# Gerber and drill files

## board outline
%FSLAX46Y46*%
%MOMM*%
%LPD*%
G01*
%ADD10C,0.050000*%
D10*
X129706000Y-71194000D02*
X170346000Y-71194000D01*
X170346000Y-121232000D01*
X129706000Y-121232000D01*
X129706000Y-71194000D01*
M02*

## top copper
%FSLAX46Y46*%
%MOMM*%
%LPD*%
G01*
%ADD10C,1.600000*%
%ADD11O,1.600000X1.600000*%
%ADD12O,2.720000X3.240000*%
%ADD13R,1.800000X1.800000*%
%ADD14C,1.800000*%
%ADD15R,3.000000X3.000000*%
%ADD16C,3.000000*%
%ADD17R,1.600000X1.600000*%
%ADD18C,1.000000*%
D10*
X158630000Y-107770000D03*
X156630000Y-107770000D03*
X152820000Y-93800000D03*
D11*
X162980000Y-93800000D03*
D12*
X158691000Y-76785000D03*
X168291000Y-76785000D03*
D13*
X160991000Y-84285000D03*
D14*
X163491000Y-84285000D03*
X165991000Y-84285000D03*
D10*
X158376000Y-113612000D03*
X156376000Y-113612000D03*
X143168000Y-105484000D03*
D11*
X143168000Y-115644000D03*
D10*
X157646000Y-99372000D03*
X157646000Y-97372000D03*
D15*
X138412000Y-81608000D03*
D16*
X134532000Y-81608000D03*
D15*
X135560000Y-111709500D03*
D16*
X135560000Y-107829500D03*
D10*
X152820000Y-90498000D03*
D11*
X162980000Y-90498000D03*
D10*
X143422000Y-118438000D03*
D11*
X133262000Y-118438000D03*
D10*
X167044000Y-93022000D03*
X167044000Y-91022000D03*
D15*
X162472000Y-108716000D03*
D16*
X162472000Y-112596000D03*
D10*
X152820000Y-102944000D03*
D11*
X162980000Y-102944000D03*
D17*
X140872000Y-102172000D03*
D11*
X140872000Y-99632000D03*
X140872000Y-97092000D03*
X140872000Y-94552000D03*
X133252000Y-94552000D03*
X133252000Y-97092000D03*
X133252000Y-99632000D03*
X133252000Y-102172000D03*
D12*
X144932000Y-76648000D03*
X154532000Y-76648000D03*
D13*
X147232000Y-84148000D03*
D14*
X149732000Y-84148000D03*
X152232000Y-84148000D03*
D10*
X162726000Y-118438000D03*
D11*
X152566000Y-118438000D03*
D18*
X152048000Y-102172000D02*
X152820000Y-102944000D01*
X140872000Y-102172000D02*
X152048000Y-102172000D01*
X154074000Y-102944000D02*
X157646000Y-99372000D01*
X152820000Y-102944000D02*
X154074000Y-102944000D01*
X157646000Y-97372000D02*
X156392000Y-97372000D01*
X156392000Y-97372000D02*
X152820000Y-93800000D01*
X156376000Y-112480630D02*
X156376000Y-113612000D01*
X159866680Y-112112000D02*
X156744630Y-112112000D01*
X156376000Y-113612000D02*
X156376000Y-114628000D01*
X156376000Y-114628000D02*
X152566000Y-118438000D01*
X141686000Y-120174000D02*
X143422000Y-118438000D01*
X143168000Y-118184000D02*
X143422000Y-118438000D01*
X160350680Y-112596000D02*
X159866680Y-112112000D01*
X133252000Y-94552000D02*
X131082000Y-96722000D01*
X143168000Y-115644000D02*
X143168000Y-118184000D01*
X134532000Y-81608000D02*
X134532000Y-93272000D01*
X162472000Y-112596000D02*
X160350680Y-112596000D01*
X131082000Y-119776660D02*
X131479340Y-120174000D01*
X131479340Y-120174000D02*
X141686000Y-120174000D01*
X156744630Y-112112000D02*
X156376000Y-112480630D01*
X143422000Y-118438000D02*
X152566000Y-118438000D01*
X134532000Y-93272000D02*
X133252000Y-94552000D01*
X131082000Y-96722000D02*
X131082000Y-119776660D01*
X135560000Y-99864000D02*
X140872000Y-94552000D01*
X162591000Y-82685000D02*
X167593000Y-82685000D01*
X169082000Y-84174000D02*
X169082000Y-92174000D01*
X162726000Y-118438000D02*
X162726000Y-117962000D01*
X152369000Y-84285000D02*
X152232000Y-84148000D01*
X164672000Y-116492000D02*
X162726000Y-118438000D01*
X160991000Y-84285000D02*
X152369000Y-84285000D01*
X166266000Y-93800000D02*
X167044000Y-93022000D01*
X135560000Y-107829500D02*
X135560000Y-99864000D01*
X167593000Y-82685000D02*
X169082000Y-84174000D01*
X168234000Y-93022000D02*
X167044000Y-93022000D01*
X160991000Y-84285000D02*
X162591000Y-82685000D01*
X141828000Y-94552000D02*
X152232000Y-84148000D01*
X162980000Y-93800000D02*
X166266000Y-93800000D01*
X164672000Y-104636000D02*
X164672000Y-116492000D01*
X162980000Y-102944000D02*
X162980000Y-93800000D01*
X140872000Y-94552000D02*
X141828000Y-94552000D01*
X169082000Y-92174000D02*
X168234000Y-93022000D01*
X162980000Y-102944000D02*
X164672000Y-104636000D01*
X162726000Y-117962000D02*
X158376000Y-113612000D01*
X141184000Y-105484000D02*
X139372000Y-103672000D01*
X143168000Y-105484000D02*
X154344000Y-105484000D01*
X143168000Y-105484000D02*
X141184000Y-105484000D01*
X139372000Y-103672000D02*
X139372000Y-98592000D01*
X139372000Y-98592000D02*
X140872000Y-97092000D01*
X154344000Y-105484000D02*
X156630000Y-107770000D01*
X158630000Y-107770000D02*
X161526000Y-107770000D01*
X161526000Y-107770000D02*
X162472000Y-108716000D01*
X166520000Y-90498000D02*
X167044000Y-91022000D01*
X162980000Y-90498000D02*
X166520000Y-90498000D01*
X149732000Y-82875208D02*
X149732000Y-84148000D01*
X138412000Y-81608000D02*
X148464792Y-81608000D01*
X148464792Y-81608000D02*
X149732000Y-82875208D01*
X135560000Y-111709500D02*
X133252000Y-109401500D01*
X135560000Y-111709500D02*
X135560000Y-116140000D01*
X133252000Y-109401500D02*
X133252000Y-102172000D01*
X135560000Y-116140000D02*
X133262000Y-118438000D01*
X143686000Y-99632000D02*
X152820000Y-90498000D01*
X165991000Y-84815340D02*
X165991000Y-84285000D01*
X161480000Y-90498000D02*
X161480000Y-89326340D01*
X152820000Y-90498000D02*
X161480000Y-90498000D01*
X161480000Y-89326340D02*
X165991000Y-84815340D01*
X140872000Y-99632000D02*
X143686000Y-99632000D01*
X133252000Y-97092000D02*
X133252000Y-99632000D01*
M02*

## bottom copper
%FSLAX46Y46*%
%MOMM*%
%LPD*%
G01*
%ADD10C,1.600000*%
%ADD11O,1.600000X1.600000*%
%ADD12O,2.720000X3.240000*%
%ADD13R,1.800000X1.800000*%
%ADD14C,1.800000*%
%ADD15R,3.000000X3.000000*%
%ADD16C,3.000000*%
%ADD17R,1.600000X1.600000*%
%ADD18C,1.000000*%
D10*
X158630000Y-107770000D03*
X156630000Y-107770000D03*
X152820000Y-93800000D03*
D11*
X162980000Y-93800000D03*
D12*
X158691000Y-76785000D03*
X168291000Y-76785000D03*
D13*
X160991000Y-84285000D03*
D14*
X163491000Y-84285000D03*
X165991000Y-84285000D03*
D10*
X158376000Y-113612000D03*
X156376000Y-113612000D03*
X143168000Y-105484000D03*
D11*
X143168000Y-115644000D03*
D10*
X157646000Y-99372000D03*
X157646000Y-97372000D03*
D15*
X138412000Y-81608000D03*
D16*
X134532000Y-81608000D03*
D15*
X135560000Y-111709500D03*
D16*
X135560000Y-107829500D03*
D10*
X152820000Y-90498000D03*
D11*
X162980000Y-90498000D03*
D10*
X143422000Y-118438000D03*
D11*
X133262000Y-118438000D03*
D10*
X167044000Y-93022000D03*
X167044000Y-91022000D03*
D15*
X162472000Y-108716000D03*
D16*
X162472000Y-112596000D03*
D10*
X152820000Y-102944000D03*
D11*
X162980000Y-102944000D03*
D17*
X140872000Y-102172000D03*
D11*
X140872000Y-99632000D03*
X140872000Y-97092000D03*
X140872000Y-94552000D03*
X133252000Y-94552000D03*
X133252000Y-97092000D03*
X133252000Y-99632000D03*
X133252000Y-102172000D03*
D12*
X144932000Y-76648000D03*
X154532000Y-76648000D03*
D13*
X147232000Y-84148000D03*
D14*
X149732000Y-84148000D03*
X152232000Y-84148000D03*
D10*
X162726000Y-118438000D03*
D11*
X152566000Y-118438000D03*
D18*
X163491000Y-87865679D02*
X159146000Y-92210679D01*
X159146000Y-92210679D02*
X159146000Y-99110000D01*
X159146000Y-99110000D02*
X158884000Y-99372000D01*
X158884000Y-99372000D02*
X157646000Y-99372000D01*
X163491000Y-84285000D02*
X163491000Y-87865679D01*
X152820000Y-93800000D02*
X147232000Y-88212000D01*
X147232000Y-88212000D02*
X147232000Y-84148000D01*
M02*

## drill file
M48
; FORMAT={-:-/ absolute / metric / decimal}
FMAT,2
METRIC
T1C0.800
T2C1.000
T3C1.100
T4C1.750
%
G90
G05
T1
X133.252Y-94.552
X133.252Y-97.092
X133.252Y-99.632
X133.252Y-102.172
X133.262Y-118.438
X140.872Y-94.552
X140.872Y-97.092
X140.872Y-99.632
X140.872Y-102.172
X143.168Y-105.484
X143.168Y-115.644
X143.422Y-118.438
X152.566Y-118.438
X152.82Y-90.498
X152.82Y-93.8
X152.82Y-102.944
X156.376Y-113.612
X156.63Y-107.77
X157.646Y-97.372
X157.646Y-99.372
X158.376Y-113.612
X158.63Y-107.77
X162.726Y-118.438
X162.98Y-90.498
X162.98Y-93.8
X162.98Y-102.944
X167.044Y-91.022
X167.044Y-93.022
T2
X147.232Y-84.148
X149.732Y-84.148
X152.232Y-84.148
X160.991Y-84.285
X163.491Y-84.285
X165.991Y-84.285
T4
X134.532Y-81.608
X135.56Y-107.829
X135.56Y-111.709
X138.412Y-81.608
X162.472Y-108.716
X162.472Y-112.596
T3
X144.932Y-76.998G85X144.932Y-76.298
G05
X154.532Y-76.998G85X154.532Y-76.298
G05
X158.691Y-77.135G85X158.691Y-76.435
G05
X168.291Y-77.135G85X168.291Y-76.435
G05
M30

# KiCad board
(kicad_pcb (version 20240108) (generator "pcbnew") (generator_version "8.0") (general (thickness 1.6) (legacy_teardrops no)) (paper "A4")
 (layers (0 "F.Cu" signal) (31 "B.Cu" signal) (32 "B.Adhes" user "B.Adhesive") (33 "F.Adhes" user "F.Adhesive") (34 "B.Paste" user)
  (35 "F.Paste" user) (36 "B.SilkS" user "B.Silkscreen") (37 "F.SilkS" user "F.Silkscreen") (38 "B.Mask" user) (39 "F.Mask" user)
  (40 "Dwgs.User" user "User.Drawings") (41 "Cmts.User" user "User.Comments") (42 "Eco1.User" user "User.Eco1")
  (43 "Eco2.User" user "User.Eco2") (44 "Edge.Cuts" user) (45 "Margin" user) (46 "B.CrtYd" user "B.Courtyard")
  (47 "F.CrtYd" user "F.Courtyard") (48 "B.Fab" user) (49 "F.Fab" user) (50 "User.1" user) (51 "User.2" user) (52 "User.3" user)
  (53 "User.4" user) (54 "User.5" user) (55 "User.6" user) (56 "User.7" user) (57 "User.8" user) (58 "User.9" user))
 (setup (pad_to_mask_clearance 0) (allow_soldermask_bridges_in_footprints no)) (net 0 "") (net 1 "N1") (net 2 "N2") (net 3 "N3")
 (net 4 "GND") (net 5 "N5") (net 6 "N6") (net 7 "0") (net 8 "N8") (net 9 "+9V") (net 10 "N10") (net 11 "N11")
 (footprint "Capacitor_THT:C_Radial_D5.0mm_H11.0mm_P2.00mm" (layer "F.Cu") (at 158.63 107.77 180)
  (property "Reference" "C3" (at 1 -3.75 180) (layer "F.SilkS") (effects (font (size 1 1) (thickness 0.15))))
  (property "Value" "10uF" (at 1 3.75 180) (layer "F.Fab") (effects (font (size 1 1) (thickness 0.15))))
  (pad "1" thru_hole circle (at 0 0 180) (size 1.6 1.6) (drill 0.8) (layers "*.Cu" "*.Mask") (remove_unused_layers no) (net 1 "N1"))
  (pad "2" thru_hole circle (at 2 0 180) (size 1.6 1.6) (drill 0.8) (layers "*.Cu" "*.Mask") (remove_unused_layers no) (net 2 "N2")))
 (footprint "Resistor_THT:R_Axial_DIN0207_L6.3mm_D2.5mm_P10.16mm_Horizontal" (layer "F.Cu") (at 152.82 93.8)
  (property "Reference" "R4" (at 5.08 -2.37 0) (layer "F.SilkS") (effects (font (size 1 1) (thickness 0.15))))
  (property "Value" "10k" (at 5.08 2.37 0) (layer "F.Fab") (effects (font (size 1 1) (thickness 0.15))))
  (pad "1" thru_hole circle (at 0 0) (size 1.6 1.6) (drill 0.8) (layers "*.Cu" "*.Mask") (remove_unused_layers no) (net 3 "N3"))
  (pad "2" thru_hole oval (at 10.16 0) (size 1.6 1.6) (drill 0.8) (layers "*.Cu" "*.Mask") (remove_unused_layers no) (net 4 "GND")))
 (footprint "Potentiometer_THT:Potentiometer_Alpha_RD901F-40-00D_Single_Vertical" (layer "F.Cu") (at 160.991 84.285 90)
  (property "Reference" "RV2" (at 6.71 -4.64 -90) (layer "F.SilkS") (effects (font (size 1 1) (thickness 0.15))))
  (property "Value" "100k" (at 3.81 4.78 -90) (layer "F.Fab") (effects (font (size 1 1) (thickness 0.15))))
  (pad "" thru_hole oval (at 7.5 -2.3 180) (size 2.72 3.24) (drill oval 1.1 1.8) (layers "*.Cu" "*.Mask") (remove_unused_layers no))
  (pad "" thru_hole oval (at 7.5 7.3 180) (size 2.72 3.24) (drill oval 1.1 1.8) (layers "*.Cu" "*.Mask") (remove_unused_layers no))
  (pad "1" thru_hole rect (at 0 0 180) (size 1.8 1.8) (drill 1) (layers "*.Cu" "*.Mask") (remove_unused_layers no) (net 4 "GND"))
  (pad "2" thru_hole circle (at 0 2.5 180) (size 1.8 1.8) (drill 1) (layers "*.Cu" "*.Mask") (remove_unused_layers no) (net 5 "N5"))
  (pad "3" thru_hole circle (at 0 5 180) (size 1.8 1.8) (drill 1) (layers "*.Cu" "*.Mask") (remove_unused_layers no) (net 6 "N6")))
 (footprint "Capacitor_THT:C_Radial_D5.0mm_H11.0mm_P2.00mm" (layer "F.Cu") (at 158.376 113.612 180)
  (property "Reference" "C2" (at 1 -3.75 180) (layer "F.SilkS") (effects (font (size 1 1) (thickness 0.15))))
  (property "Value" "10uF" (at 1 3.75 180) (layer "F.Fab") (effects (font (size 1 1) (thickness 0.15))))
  (pad "1" thru_hole circle (at 0 0 180) (size 1.6 1.6) (drill 0.8) (layers "*.Cu" "*.Mask") (remove_unused_layers no) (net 4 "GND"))
  (pad "2" thru_hole circle (at 2 0 180) (size 1.6 1.6) (drill 0.8) (layers "*.Cu" "*.Mask") (remove_unused_layers no) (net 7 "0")))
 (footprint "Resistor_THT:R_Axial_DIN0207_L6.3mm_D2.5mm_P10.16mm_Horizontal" (layer "F.Cu") (at 143.168 105.484 -90)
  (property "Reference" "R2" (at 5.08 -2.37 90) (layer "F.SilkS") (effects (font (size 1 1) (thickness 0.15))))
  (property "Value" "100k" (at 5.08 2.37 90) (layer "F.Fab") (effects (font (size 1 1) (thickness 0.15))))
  (pad "1" thru_hole circle (at 0 0 270) (size 1.6 1.6) (drill 0.8) (layers "*.Cu" "*.Mask") (remove_unused_layers no) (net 2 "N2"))
  (pad "2" thru_hole oval (at 10.16 0 270) (size 1.6 1.6) (drill 0.8) (layers "*.Cu" "*.Mask") (remove_unused_layers no) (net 7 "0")))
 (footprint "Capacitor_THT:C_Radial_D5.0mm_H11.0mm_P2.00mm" (layer "F.Cu") (at 157.646 99.372 90)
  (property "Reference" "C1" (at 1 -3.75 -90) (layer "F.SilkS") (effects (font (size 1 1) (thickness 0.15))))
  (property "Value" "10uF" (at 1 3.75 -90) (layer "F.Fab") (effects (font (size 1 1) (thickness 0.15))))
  (pad "1" thru_hole circle (at 0 0 90) (size 1.6 1.6) (drill 0.8) (layers "*.Cu" "*.Mask") (remove_unused_layers no) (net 5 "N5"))
  (pad "2" thru_hole circle (at 2 0 90) (size 1.6 1.6) (drill 0.8) (layers "*.Cu" "*.Mask") (remove_unused_layers no) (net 3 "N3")))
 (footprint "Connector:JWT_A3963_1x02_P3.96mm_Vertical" (layer "F.Cu") (at 138.412 81.608 180)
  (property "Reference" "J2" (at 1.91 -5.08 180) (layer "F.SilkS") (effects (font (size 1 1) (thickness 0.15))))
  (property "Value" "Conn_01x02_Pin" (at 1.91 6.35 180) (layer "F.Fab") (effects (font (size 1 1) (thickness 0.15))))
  (pad "1" thru_hole rect (at 0 0 180) (size 3 3) (drill 1.75) (layers "*.Cu" "*.Mask") (remove_unused_layers no) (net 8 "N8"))
  (pad "2" thru_hole circle (at 3.88 0 180) (size 3 3) (drill 1.75) (layers "*.Cu" "*.Mask") (remove_unused_layers no) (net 7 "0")))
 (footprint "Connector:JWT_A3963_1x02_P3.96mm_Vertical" (layer "F.Cu") (at 135.56 111.7095 90)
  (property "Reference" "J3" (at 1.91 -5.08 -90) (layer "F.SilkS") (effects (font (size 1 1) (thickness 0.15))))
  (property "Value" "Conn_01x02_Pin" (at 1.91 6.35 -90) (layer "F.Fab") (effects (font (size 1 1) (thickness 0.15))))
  (pad "1" thru_hole rect (at 0 0 90) (size 3 3) (drill 1.75) (layers "*.Cu" "*.Mask") (remove_unused_layers no) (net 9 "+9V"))
  (pad "2" thru_hole circle (at 3.88 0 90) (size 3 3) (drill 1.75) (layers "*.Cu" "*.Mask") (remove_unused_layers no) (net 4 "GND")))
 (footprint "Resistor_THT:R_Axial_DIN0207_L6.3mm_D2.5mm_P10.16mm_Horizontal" (layer "F.Cu") (at 152.82 90.498)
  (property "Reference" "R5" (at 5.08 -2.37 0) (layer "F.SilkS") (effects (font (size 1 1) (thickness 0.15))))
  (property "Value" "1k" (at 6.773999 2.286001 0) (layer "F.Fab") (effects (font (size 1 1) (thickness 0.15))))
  (pad "1" thru_hole circle (at 0 0) (size 1.6 1.6) (drill 0.8) (layers "*.Cu" "*.Mask") (remove_unused_layers no) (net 6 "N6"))
  (pad "2" thru_hole oval (at 10.16 0) (size 1.6 1.6) (drill 0.8) (layers "*.Cu" "*.Mask") (remove_unused_layers no) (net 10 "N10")))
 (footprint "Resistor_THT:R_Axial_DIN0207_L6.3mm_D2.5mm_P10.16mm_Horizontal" (layer "F.Cu") (at 143.422 118.438 180)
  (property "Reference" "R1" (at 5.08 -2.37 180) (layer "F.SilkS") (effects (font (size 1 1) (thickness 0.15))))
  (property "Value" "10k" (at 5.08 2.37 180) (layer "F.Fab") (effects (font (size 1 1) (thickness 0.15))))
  (pad "1" thru_hole circle (at 0 0 180) (size 1.6 1.6) (drill 0.8) (layers "*.Cu" "*.Mask") (remove_unused_layers no) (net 7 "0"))
  (pad "2" thru_hole oval (at 10.16 0 180) (size 1.6 1.6) (drill 0.8) (layers "*.Cu" "*.Mask") (remove_unused_layers no) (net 9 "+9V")))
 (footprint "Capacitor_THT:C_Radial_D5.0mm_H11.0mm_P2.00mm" (layer "F.Cu") (at 167.044 93.022 90)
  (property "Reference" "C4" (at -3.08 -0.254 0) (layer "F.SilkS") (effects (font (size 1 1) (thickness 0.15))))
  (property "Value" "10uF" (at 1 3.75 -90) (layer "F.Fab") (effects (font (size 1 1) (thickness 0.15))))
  (pad "1" thru_hole circle (at 0 0 90) (size 1.6 1.6) (drill 0.8) (layers "*.Cu" "*.Mask") (remove_unused_layers no) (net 4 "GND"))
  (pad "2" thru_hole circle (at 2 0 90) (size 1.6 1.6) (drill 0.8) (layers "*.Cu" "*.Mask") (remove_unused_layers no) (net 10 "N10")))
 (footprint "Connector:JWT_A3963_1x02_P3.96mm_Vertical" (layer "F.Cu") (at 162.472 108.716 -90)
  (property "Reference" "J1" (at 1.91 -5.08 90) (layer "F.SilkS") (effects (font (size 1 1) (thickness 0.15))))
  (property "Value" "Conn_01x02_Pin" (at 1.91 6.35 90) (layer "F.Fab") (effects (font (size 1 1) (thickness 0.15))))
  (pad "1" thru_hole rect (at 0 0 270) (size 3 3) (drill 1.75) (layers "*.Cu" "*.Mask") (remove_unused_layers no) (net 1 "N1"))
  (pad "2" thru_hole circle (at 3.88 0 270) (size 3 3) (drill 1.75) (layers "*.Cu" "*.Mask") (remove_unused_layers no) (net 7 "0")))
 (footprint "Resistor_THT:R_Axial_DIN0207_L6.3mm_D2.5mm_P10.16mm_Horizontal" (layer "F.Cu") (at 152.82 102.944)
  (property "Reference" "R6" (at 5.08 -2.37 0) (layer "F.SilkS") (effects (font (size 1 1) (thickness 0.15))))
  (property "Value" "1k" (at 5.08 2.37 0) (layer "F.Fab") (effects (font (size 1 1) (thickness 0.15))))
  (pad "1" thru_hole circle (at 0 0) (size 1.6 1.6) (drill 0.8) (layers "*.Cu" "*.Mask") (remove_unused_layers no) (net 5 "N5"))
  (pad "2" thru_hole oval (at 10.16 0) (size 1.6 1.6) (drill 0.8) (layers "*.Cu" "*.Mask") (remove_unused_layers no) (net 4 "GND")))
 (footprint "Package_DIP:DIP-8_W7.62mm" (layer "F.Cu") (at 140.872 102.172 180)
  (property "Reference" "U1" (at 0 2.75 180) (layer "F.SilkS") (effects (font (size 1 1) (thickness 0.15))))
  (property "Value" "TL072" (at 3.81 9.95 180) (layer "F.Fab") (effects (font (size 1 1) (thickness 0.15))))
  (pad "1" thru_hole rect (at 0 0 180) (size 1.6 1.6) (drill 0.8) (layers "*.Cu" "*.Mask") (remove_unused_layers no) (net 5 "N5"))
  (pad "2" thru_hole oval (at 0 2.54 180) (size 1.6 1.6) (drill 0.8) (layers "*.Cu" "*.Mask") (remove_unused_layers no) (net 6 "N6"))
  (pad "3" thru_hole oval (at 0 5.08 180) (size 1.6 1.6) (drill 0.8) (layers "*.Cu" "*.Mask") (remove_unused_layers no) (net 2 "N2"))
  (pad "4" thru_hole oval (at 0 7.62 180) (size 1.6 1.6) (drill 0.8) (layers "*.Cu" "*.Mask") (remove_unused_layers no) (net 4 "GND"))
  (pad "5" thru_hole oval (at 7.62 7.62 180) (size 1.6 1.6) (drill 0.8) (layers "*.Cu" "*.Mask") (remove_unused_layers no) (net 7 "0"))
  (pad "6" thru_hole oval (at 7.62 5.08 180) (size 1.6 1.6) (drill 0.8) (layers "*.Cu" "*.Mask") (remove_unused_layers no) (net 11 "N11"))
  (pad "7" thru_hole oval (at 7.62 2.54 180) (size 1.6 1.6) (drill 0.8) (layers "*.Cu" "*.Mask") (remove_unused_layers no) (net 11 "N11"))
  (pad "8" thru_hole oval (at 7.62 0 180) (size 1.6 1.6) (drill 0.8) (layers "*.Cu" "*.Mask") (remove_unused_layers no) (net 9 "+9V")))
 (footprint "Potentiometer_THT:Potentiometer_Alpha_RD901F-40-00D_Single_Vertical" (layer "F.Cu") (at 147.232 84.148 90)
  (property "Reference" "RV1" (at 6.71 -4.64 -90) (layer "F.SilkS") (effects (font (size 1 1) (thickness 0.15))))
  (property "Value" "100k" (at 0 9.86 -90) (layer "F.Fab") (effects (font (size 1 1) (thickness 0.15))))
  (pad "" thru_hole oval (at 7.5 -2.3 180) (size 2.72 3.24) (drill oval 1.1 1.8) (layers "*.Cu" "*.Mask") (remove_unused_layers no))
  (pad "" thru_hole oval (at 7.5 7.3 180) (size 2.72 3.24) (drill oval 1.1 1.8) (layers "*.Cu" "*.Mask") (remove_unused_layers no))
  (pad "1" thru_hole rect (at 0 0 180) (size 1.8 1.8) (drill 1) (layers "*.Cu" "*.Mask") (remove_unused_layers no) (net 3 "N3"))
  (pad "2" thru_hole circle (at 0 2.5 180) (size 1.8 1.8) (drill 1) (layers "*.Cu" "*.Mask") (remove_unused_layers no) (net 8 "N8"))
  (pad "3" thru_hole circle (at 0 5 180) (size 1.8 1.8) (drill 1) (layers "*.Cu" "*.Mask") (remove_unused_layers no) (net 4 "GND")))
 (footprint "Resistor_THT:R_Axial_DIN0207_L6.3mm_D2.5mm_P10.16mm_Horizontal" (layer "F.Cu") (at 162.726 118.438 180)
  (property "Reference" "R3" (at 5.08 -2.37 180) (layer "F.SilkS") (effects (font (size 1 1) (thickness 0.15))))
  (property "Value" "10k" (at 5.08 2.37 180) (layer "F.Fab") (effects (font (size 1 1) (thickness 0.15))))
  (pad "1" thru_hole circle (at 0 0 180) (size 1.6 1.6) (drill 0.8) (layers "*.Cu" "*.Mask") (remove_unused_layers no) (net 4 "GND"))
  (pad "2" thru_hole oval (at 10.16 0 180) (size 1.6 1.6) (drill 0.8) (layers "*.Cu" "*.Mask") (remove_unused_layers no) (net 7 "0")))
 (gr_rect (start 129.706 71.194) (end 170.346 121.232) (stroke (width 0.05) (type default)) (fill none) (layer "Edge.Cuts"))
 (segment (start 152.048 102.172) (end 152.82 102.944) (width 1) (layer "F.Cu") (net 5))
 (segment (start 140.872 102.172) (end 152.048 102.172) (width 1) (layer "F.Cu") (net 5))
 (segment (start 154.074 102.944) (end 157.646 99.372) (width 1) (layer "F.Cu") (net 5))
 (segment (start 152.82 102.944) (end 154.074 102.944) (width 1) (layer "F.Cu") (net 5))
 (segment (start 163.491 87.865679) (end 159.146 92.210679) (width 1) (layer "B.Cu") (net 5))
 (segment (start 159.146 92.210679) (end 159.146 99.11) (width 1) (layer "B.Cu") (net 5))
 (segment (start 159.146 99.11) (end 158.884 99.372) (width 1) (layer "B.Cu") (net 5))
 (segment (start 158.884 99.372) (end 157.646 99.372) (width 1) (layer "B.Cu") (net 5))
 (segment (start 163.491 84.285) (end 163.491 87.865679) (width 1) (layer "B.Cu") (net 5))
 (segment (start 157.646 97.372) (end 156.392 97.372) (width 1) (layer "F.Cu") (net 3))
 (segment (start 156.392 97.372) (end 152.82 93.8) (width 1) (layer "F.Cu") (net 3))
 (segment (start 152.82 93.8) (end 147.232 88.212) (width 1) (layer "B.Cu") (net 3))
 (segment (start 147.232 88.212) (end 147.232 84.148) (width 1) (layer "B.Cu") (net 3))
 (segment (start 156.376 112.48063) (end 156.376 113.612) (width 1) (layer "F.Cu") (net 7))
 (segment (start 159.86668 112.112) (end 156.74463 112.112) (width 1) (layer "F.Cu") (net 7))
 (segment (start 156.376 113.612) (end 156.376 114.628) (width 1) (layer "F.Cu") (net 7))
 (segment (start 156.376 114.628) (end 152.566 118.438) (width 1) (layer "F.Cu") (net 7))
 (segment (start 141.686 120.174) (end 143.422 118.438) (width 1) (layer "F.Cu") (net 7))
 (segment (start 143.168 118.184) (end 143.422 118.438) (width 1) (layer "F.Cu") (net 7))
 (segment (start 160.35068 112.596) (end 159.86668 112.112) (width 1) (layer "F.Cu") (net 7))
 (segment (start 133.252 94.552) (end 131.082 96.722) (width 1) (layer "F.Cu") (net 7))
 (segment (start 143.168 115.644) (end 143.168 118.184) (width 1) (layer "F.Cu") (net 7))
 (segment (start 134.532 81.608) (end 134.532 93.272) (width 1) (layer "F.Cu") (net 7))
 (segment (start 162.472 112.596) (end 160.35068 112.596) (width 1) (layer "F.Cu") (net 7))
 (segment (start 131.082 119.77666) (end 131.47934 120.174) (width 1) (layer "F.Cu") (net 7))
 (segment (start 131.47934 120.174) (end 141.686 120.174) (width 1) (layer "F.Cu") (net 7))
 (segment (start 156.74463 112.112) (end 156.376 112.48063) (width 1) (layer "F.Cu") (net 7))
 (segment (start 143.422 118.438) (end 152.566 118.438) (width 1) (layer "F.Cu") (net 7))
 (segment (start 134.532 93.272) (end 133.252 94.552) (width 1) (layer "F.Cu") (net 7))
 (segment (start 131.082 96.722) (end 131.082 119.77666) (width 1) (layer "F.Cu") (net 7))
 (segment (start 135.56 99.864) (end 140.872 94.552) (width 1) (layer "F.Cu") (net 4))
 (segment (start 162.591 82.685) (end 167.593 82.685) (width 1) (layer "F.Cu") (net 4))
 (segment (start 169.082 84.174) (end 169.082 92.174) (width 1) (layer "F.Cu") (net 4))
 (segment (start 162.726 118.438) (end 162.726 117.962) (width 1) (layer "F.Cu") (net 4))
 (segment (start 152.369 84.285) (end 152.232 84.148) (width 1) (layer "F.Cu") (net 4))
 (segment (start 164.672 116.492) (end 162.726 118.438) (width 1) (layer "F.Cu") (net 4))
 (segment (start 160.991 84.285) (end 152.369 84.285) (width 1) (layer "F.Cu") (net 4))
 (segment (start 166.266 93.8) (end 167.044 93.022) (width 1) (layer "F.Cu") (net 4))
 (segment (start 135.56 107.8295) (end 135.56 99.864) (width 1) (layer "F.Cu") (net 4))
 (segment (start 167.593 82.685) (end 169.082 84.174) (width 1) (layer "F.Cu") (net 4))
 (segment (start 168.234 93.022) (end 167.044 93.022) (width 1) (layer "F.Cu") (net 4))
 (segment (start 160.991 84.285) (end 162.591 82.685) (width 1) (layer "F.Cu") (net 4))
 (segment (start 141.828 94.552) (end 152.232 84.148) (width 1) (layer "F.Cu") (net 4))
 (segment (start 162.98 93.8) (end 166.266 93.8) (width 1) (layer "F.Cu") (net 4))
 (segment (start 164.672 104.636) (end 164.672 116.492) (width 1) (layer "F.Cu") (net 4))
 (segment (start 162.98 102.944) (end 162.98 93.8) (width 1) (layer "F.Cu") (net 4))
 (segment (start 140.872 94.552) (end 141.828 94.552) (width 1) (layer "F.Cu") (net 4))
 (segment (start 169.082 92.174) (end 168.234 93.022) (width 1) (layer "F.Cu") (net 4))
 (segment (start 162.98 102.944) (end 164.672 104.636) (width 1) (layer "F.Cu") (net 4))
 (segment (start 162.726 117.962) (end 158.376 113.612) (width 1) (layer "F.Cu") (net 4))
 (segment (start 141.184 105.484) (end 139.372 103.672) (width 1) (layer "F.Cu") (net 2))
 (segment (start 143.168 105.484) (end 154.344 105.484) (width 1) (layer "F.Cu") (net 2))
 (segment (start 143.168 105.484) (end 141.184 105.484) (width 1) (layer "F.Cu") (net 2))
 (segment (start 139.372 103.672) (end 139.372 98.592) (width 1) (layer "F.Cu") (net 2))
 (segment (start 139.372 98.592) (end 140.872 97.092) (width 1) (layer "F.Cu") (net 2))
 (segment (start 154.344 105.484) (end 156.63 107.77) (width 1) (layer "F.Cu") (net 2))
 (segment (start 158.63 107.77) (end 161.526 107.77) (width 1) (layer "F.Cu") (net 1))
 (segment (start 161.526 107.77) (end 162.472 108.716) (width 1) (layer "F.Cu") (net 1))
 (segment (start 166.52 90.498) (end 167.044 91.022) (width 1) (layer "F.Cu") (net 10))
 (segment (start 162.98 90.498) (end 166.52 90.498) (width 1) (layer "F.Cu") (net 10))
 (segment (start 149.732 82.875208) (end 149.732 84.148) (width 1) (layer "F.Cu") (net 8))
 (segment (start 138.412 81.608) (end 148.464792 81.608) (width 1) (layer "F.Cu") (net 8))
 (segment (start 148.464792 81.608) (end 149.732 82.875208) (width 1) (layer "F.Cu") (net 8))
 (segment (start 135.56 111.7095) (end 133.252 109.4015) (width 1) (layer "F.Cu") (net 9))
 (segment (start 135.56 111.7095) (end 135.56 116.14) (width 1) (layer "F.Cu") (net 9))
 (segment (start 133.252 109.4015) (end 133.252 102.172) (width 1) (layer "F.Cu") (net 9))
 (segment (start 135.56 116.14) (end 133.262 118.438) (width 1) (layer "F.Cu") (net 9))
 (segment (start 143.686 99.632) (end 152.82 90.498) (width 1) (layer "F.Cu") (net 6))
 (segment (start 165.991 84.81534) (end 165.991 84.285) (width 1) (layer "F.Cu") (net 6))
 (segment (start 161.48 90.498) (end 161.48 89.32634) (width 1) (layer "F.Cu") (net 6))
 (segment (start 152.82 90.498) (end 161.48 90.498) (width 1) (layer "F.Cu") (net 6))
 (segment (start 161.48 89.32634) (end 165.991 84.81534) (width 1) (layer "F.Cu") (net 6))
 (segment (start 140.872 99.632) (end 143.686 99.632) (width 1) (layer "F.Cu") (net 6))
 (segment (start 133.252 97.092) (end 133.252 99.632) (width 1) (layer "F.Cu") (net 11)))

